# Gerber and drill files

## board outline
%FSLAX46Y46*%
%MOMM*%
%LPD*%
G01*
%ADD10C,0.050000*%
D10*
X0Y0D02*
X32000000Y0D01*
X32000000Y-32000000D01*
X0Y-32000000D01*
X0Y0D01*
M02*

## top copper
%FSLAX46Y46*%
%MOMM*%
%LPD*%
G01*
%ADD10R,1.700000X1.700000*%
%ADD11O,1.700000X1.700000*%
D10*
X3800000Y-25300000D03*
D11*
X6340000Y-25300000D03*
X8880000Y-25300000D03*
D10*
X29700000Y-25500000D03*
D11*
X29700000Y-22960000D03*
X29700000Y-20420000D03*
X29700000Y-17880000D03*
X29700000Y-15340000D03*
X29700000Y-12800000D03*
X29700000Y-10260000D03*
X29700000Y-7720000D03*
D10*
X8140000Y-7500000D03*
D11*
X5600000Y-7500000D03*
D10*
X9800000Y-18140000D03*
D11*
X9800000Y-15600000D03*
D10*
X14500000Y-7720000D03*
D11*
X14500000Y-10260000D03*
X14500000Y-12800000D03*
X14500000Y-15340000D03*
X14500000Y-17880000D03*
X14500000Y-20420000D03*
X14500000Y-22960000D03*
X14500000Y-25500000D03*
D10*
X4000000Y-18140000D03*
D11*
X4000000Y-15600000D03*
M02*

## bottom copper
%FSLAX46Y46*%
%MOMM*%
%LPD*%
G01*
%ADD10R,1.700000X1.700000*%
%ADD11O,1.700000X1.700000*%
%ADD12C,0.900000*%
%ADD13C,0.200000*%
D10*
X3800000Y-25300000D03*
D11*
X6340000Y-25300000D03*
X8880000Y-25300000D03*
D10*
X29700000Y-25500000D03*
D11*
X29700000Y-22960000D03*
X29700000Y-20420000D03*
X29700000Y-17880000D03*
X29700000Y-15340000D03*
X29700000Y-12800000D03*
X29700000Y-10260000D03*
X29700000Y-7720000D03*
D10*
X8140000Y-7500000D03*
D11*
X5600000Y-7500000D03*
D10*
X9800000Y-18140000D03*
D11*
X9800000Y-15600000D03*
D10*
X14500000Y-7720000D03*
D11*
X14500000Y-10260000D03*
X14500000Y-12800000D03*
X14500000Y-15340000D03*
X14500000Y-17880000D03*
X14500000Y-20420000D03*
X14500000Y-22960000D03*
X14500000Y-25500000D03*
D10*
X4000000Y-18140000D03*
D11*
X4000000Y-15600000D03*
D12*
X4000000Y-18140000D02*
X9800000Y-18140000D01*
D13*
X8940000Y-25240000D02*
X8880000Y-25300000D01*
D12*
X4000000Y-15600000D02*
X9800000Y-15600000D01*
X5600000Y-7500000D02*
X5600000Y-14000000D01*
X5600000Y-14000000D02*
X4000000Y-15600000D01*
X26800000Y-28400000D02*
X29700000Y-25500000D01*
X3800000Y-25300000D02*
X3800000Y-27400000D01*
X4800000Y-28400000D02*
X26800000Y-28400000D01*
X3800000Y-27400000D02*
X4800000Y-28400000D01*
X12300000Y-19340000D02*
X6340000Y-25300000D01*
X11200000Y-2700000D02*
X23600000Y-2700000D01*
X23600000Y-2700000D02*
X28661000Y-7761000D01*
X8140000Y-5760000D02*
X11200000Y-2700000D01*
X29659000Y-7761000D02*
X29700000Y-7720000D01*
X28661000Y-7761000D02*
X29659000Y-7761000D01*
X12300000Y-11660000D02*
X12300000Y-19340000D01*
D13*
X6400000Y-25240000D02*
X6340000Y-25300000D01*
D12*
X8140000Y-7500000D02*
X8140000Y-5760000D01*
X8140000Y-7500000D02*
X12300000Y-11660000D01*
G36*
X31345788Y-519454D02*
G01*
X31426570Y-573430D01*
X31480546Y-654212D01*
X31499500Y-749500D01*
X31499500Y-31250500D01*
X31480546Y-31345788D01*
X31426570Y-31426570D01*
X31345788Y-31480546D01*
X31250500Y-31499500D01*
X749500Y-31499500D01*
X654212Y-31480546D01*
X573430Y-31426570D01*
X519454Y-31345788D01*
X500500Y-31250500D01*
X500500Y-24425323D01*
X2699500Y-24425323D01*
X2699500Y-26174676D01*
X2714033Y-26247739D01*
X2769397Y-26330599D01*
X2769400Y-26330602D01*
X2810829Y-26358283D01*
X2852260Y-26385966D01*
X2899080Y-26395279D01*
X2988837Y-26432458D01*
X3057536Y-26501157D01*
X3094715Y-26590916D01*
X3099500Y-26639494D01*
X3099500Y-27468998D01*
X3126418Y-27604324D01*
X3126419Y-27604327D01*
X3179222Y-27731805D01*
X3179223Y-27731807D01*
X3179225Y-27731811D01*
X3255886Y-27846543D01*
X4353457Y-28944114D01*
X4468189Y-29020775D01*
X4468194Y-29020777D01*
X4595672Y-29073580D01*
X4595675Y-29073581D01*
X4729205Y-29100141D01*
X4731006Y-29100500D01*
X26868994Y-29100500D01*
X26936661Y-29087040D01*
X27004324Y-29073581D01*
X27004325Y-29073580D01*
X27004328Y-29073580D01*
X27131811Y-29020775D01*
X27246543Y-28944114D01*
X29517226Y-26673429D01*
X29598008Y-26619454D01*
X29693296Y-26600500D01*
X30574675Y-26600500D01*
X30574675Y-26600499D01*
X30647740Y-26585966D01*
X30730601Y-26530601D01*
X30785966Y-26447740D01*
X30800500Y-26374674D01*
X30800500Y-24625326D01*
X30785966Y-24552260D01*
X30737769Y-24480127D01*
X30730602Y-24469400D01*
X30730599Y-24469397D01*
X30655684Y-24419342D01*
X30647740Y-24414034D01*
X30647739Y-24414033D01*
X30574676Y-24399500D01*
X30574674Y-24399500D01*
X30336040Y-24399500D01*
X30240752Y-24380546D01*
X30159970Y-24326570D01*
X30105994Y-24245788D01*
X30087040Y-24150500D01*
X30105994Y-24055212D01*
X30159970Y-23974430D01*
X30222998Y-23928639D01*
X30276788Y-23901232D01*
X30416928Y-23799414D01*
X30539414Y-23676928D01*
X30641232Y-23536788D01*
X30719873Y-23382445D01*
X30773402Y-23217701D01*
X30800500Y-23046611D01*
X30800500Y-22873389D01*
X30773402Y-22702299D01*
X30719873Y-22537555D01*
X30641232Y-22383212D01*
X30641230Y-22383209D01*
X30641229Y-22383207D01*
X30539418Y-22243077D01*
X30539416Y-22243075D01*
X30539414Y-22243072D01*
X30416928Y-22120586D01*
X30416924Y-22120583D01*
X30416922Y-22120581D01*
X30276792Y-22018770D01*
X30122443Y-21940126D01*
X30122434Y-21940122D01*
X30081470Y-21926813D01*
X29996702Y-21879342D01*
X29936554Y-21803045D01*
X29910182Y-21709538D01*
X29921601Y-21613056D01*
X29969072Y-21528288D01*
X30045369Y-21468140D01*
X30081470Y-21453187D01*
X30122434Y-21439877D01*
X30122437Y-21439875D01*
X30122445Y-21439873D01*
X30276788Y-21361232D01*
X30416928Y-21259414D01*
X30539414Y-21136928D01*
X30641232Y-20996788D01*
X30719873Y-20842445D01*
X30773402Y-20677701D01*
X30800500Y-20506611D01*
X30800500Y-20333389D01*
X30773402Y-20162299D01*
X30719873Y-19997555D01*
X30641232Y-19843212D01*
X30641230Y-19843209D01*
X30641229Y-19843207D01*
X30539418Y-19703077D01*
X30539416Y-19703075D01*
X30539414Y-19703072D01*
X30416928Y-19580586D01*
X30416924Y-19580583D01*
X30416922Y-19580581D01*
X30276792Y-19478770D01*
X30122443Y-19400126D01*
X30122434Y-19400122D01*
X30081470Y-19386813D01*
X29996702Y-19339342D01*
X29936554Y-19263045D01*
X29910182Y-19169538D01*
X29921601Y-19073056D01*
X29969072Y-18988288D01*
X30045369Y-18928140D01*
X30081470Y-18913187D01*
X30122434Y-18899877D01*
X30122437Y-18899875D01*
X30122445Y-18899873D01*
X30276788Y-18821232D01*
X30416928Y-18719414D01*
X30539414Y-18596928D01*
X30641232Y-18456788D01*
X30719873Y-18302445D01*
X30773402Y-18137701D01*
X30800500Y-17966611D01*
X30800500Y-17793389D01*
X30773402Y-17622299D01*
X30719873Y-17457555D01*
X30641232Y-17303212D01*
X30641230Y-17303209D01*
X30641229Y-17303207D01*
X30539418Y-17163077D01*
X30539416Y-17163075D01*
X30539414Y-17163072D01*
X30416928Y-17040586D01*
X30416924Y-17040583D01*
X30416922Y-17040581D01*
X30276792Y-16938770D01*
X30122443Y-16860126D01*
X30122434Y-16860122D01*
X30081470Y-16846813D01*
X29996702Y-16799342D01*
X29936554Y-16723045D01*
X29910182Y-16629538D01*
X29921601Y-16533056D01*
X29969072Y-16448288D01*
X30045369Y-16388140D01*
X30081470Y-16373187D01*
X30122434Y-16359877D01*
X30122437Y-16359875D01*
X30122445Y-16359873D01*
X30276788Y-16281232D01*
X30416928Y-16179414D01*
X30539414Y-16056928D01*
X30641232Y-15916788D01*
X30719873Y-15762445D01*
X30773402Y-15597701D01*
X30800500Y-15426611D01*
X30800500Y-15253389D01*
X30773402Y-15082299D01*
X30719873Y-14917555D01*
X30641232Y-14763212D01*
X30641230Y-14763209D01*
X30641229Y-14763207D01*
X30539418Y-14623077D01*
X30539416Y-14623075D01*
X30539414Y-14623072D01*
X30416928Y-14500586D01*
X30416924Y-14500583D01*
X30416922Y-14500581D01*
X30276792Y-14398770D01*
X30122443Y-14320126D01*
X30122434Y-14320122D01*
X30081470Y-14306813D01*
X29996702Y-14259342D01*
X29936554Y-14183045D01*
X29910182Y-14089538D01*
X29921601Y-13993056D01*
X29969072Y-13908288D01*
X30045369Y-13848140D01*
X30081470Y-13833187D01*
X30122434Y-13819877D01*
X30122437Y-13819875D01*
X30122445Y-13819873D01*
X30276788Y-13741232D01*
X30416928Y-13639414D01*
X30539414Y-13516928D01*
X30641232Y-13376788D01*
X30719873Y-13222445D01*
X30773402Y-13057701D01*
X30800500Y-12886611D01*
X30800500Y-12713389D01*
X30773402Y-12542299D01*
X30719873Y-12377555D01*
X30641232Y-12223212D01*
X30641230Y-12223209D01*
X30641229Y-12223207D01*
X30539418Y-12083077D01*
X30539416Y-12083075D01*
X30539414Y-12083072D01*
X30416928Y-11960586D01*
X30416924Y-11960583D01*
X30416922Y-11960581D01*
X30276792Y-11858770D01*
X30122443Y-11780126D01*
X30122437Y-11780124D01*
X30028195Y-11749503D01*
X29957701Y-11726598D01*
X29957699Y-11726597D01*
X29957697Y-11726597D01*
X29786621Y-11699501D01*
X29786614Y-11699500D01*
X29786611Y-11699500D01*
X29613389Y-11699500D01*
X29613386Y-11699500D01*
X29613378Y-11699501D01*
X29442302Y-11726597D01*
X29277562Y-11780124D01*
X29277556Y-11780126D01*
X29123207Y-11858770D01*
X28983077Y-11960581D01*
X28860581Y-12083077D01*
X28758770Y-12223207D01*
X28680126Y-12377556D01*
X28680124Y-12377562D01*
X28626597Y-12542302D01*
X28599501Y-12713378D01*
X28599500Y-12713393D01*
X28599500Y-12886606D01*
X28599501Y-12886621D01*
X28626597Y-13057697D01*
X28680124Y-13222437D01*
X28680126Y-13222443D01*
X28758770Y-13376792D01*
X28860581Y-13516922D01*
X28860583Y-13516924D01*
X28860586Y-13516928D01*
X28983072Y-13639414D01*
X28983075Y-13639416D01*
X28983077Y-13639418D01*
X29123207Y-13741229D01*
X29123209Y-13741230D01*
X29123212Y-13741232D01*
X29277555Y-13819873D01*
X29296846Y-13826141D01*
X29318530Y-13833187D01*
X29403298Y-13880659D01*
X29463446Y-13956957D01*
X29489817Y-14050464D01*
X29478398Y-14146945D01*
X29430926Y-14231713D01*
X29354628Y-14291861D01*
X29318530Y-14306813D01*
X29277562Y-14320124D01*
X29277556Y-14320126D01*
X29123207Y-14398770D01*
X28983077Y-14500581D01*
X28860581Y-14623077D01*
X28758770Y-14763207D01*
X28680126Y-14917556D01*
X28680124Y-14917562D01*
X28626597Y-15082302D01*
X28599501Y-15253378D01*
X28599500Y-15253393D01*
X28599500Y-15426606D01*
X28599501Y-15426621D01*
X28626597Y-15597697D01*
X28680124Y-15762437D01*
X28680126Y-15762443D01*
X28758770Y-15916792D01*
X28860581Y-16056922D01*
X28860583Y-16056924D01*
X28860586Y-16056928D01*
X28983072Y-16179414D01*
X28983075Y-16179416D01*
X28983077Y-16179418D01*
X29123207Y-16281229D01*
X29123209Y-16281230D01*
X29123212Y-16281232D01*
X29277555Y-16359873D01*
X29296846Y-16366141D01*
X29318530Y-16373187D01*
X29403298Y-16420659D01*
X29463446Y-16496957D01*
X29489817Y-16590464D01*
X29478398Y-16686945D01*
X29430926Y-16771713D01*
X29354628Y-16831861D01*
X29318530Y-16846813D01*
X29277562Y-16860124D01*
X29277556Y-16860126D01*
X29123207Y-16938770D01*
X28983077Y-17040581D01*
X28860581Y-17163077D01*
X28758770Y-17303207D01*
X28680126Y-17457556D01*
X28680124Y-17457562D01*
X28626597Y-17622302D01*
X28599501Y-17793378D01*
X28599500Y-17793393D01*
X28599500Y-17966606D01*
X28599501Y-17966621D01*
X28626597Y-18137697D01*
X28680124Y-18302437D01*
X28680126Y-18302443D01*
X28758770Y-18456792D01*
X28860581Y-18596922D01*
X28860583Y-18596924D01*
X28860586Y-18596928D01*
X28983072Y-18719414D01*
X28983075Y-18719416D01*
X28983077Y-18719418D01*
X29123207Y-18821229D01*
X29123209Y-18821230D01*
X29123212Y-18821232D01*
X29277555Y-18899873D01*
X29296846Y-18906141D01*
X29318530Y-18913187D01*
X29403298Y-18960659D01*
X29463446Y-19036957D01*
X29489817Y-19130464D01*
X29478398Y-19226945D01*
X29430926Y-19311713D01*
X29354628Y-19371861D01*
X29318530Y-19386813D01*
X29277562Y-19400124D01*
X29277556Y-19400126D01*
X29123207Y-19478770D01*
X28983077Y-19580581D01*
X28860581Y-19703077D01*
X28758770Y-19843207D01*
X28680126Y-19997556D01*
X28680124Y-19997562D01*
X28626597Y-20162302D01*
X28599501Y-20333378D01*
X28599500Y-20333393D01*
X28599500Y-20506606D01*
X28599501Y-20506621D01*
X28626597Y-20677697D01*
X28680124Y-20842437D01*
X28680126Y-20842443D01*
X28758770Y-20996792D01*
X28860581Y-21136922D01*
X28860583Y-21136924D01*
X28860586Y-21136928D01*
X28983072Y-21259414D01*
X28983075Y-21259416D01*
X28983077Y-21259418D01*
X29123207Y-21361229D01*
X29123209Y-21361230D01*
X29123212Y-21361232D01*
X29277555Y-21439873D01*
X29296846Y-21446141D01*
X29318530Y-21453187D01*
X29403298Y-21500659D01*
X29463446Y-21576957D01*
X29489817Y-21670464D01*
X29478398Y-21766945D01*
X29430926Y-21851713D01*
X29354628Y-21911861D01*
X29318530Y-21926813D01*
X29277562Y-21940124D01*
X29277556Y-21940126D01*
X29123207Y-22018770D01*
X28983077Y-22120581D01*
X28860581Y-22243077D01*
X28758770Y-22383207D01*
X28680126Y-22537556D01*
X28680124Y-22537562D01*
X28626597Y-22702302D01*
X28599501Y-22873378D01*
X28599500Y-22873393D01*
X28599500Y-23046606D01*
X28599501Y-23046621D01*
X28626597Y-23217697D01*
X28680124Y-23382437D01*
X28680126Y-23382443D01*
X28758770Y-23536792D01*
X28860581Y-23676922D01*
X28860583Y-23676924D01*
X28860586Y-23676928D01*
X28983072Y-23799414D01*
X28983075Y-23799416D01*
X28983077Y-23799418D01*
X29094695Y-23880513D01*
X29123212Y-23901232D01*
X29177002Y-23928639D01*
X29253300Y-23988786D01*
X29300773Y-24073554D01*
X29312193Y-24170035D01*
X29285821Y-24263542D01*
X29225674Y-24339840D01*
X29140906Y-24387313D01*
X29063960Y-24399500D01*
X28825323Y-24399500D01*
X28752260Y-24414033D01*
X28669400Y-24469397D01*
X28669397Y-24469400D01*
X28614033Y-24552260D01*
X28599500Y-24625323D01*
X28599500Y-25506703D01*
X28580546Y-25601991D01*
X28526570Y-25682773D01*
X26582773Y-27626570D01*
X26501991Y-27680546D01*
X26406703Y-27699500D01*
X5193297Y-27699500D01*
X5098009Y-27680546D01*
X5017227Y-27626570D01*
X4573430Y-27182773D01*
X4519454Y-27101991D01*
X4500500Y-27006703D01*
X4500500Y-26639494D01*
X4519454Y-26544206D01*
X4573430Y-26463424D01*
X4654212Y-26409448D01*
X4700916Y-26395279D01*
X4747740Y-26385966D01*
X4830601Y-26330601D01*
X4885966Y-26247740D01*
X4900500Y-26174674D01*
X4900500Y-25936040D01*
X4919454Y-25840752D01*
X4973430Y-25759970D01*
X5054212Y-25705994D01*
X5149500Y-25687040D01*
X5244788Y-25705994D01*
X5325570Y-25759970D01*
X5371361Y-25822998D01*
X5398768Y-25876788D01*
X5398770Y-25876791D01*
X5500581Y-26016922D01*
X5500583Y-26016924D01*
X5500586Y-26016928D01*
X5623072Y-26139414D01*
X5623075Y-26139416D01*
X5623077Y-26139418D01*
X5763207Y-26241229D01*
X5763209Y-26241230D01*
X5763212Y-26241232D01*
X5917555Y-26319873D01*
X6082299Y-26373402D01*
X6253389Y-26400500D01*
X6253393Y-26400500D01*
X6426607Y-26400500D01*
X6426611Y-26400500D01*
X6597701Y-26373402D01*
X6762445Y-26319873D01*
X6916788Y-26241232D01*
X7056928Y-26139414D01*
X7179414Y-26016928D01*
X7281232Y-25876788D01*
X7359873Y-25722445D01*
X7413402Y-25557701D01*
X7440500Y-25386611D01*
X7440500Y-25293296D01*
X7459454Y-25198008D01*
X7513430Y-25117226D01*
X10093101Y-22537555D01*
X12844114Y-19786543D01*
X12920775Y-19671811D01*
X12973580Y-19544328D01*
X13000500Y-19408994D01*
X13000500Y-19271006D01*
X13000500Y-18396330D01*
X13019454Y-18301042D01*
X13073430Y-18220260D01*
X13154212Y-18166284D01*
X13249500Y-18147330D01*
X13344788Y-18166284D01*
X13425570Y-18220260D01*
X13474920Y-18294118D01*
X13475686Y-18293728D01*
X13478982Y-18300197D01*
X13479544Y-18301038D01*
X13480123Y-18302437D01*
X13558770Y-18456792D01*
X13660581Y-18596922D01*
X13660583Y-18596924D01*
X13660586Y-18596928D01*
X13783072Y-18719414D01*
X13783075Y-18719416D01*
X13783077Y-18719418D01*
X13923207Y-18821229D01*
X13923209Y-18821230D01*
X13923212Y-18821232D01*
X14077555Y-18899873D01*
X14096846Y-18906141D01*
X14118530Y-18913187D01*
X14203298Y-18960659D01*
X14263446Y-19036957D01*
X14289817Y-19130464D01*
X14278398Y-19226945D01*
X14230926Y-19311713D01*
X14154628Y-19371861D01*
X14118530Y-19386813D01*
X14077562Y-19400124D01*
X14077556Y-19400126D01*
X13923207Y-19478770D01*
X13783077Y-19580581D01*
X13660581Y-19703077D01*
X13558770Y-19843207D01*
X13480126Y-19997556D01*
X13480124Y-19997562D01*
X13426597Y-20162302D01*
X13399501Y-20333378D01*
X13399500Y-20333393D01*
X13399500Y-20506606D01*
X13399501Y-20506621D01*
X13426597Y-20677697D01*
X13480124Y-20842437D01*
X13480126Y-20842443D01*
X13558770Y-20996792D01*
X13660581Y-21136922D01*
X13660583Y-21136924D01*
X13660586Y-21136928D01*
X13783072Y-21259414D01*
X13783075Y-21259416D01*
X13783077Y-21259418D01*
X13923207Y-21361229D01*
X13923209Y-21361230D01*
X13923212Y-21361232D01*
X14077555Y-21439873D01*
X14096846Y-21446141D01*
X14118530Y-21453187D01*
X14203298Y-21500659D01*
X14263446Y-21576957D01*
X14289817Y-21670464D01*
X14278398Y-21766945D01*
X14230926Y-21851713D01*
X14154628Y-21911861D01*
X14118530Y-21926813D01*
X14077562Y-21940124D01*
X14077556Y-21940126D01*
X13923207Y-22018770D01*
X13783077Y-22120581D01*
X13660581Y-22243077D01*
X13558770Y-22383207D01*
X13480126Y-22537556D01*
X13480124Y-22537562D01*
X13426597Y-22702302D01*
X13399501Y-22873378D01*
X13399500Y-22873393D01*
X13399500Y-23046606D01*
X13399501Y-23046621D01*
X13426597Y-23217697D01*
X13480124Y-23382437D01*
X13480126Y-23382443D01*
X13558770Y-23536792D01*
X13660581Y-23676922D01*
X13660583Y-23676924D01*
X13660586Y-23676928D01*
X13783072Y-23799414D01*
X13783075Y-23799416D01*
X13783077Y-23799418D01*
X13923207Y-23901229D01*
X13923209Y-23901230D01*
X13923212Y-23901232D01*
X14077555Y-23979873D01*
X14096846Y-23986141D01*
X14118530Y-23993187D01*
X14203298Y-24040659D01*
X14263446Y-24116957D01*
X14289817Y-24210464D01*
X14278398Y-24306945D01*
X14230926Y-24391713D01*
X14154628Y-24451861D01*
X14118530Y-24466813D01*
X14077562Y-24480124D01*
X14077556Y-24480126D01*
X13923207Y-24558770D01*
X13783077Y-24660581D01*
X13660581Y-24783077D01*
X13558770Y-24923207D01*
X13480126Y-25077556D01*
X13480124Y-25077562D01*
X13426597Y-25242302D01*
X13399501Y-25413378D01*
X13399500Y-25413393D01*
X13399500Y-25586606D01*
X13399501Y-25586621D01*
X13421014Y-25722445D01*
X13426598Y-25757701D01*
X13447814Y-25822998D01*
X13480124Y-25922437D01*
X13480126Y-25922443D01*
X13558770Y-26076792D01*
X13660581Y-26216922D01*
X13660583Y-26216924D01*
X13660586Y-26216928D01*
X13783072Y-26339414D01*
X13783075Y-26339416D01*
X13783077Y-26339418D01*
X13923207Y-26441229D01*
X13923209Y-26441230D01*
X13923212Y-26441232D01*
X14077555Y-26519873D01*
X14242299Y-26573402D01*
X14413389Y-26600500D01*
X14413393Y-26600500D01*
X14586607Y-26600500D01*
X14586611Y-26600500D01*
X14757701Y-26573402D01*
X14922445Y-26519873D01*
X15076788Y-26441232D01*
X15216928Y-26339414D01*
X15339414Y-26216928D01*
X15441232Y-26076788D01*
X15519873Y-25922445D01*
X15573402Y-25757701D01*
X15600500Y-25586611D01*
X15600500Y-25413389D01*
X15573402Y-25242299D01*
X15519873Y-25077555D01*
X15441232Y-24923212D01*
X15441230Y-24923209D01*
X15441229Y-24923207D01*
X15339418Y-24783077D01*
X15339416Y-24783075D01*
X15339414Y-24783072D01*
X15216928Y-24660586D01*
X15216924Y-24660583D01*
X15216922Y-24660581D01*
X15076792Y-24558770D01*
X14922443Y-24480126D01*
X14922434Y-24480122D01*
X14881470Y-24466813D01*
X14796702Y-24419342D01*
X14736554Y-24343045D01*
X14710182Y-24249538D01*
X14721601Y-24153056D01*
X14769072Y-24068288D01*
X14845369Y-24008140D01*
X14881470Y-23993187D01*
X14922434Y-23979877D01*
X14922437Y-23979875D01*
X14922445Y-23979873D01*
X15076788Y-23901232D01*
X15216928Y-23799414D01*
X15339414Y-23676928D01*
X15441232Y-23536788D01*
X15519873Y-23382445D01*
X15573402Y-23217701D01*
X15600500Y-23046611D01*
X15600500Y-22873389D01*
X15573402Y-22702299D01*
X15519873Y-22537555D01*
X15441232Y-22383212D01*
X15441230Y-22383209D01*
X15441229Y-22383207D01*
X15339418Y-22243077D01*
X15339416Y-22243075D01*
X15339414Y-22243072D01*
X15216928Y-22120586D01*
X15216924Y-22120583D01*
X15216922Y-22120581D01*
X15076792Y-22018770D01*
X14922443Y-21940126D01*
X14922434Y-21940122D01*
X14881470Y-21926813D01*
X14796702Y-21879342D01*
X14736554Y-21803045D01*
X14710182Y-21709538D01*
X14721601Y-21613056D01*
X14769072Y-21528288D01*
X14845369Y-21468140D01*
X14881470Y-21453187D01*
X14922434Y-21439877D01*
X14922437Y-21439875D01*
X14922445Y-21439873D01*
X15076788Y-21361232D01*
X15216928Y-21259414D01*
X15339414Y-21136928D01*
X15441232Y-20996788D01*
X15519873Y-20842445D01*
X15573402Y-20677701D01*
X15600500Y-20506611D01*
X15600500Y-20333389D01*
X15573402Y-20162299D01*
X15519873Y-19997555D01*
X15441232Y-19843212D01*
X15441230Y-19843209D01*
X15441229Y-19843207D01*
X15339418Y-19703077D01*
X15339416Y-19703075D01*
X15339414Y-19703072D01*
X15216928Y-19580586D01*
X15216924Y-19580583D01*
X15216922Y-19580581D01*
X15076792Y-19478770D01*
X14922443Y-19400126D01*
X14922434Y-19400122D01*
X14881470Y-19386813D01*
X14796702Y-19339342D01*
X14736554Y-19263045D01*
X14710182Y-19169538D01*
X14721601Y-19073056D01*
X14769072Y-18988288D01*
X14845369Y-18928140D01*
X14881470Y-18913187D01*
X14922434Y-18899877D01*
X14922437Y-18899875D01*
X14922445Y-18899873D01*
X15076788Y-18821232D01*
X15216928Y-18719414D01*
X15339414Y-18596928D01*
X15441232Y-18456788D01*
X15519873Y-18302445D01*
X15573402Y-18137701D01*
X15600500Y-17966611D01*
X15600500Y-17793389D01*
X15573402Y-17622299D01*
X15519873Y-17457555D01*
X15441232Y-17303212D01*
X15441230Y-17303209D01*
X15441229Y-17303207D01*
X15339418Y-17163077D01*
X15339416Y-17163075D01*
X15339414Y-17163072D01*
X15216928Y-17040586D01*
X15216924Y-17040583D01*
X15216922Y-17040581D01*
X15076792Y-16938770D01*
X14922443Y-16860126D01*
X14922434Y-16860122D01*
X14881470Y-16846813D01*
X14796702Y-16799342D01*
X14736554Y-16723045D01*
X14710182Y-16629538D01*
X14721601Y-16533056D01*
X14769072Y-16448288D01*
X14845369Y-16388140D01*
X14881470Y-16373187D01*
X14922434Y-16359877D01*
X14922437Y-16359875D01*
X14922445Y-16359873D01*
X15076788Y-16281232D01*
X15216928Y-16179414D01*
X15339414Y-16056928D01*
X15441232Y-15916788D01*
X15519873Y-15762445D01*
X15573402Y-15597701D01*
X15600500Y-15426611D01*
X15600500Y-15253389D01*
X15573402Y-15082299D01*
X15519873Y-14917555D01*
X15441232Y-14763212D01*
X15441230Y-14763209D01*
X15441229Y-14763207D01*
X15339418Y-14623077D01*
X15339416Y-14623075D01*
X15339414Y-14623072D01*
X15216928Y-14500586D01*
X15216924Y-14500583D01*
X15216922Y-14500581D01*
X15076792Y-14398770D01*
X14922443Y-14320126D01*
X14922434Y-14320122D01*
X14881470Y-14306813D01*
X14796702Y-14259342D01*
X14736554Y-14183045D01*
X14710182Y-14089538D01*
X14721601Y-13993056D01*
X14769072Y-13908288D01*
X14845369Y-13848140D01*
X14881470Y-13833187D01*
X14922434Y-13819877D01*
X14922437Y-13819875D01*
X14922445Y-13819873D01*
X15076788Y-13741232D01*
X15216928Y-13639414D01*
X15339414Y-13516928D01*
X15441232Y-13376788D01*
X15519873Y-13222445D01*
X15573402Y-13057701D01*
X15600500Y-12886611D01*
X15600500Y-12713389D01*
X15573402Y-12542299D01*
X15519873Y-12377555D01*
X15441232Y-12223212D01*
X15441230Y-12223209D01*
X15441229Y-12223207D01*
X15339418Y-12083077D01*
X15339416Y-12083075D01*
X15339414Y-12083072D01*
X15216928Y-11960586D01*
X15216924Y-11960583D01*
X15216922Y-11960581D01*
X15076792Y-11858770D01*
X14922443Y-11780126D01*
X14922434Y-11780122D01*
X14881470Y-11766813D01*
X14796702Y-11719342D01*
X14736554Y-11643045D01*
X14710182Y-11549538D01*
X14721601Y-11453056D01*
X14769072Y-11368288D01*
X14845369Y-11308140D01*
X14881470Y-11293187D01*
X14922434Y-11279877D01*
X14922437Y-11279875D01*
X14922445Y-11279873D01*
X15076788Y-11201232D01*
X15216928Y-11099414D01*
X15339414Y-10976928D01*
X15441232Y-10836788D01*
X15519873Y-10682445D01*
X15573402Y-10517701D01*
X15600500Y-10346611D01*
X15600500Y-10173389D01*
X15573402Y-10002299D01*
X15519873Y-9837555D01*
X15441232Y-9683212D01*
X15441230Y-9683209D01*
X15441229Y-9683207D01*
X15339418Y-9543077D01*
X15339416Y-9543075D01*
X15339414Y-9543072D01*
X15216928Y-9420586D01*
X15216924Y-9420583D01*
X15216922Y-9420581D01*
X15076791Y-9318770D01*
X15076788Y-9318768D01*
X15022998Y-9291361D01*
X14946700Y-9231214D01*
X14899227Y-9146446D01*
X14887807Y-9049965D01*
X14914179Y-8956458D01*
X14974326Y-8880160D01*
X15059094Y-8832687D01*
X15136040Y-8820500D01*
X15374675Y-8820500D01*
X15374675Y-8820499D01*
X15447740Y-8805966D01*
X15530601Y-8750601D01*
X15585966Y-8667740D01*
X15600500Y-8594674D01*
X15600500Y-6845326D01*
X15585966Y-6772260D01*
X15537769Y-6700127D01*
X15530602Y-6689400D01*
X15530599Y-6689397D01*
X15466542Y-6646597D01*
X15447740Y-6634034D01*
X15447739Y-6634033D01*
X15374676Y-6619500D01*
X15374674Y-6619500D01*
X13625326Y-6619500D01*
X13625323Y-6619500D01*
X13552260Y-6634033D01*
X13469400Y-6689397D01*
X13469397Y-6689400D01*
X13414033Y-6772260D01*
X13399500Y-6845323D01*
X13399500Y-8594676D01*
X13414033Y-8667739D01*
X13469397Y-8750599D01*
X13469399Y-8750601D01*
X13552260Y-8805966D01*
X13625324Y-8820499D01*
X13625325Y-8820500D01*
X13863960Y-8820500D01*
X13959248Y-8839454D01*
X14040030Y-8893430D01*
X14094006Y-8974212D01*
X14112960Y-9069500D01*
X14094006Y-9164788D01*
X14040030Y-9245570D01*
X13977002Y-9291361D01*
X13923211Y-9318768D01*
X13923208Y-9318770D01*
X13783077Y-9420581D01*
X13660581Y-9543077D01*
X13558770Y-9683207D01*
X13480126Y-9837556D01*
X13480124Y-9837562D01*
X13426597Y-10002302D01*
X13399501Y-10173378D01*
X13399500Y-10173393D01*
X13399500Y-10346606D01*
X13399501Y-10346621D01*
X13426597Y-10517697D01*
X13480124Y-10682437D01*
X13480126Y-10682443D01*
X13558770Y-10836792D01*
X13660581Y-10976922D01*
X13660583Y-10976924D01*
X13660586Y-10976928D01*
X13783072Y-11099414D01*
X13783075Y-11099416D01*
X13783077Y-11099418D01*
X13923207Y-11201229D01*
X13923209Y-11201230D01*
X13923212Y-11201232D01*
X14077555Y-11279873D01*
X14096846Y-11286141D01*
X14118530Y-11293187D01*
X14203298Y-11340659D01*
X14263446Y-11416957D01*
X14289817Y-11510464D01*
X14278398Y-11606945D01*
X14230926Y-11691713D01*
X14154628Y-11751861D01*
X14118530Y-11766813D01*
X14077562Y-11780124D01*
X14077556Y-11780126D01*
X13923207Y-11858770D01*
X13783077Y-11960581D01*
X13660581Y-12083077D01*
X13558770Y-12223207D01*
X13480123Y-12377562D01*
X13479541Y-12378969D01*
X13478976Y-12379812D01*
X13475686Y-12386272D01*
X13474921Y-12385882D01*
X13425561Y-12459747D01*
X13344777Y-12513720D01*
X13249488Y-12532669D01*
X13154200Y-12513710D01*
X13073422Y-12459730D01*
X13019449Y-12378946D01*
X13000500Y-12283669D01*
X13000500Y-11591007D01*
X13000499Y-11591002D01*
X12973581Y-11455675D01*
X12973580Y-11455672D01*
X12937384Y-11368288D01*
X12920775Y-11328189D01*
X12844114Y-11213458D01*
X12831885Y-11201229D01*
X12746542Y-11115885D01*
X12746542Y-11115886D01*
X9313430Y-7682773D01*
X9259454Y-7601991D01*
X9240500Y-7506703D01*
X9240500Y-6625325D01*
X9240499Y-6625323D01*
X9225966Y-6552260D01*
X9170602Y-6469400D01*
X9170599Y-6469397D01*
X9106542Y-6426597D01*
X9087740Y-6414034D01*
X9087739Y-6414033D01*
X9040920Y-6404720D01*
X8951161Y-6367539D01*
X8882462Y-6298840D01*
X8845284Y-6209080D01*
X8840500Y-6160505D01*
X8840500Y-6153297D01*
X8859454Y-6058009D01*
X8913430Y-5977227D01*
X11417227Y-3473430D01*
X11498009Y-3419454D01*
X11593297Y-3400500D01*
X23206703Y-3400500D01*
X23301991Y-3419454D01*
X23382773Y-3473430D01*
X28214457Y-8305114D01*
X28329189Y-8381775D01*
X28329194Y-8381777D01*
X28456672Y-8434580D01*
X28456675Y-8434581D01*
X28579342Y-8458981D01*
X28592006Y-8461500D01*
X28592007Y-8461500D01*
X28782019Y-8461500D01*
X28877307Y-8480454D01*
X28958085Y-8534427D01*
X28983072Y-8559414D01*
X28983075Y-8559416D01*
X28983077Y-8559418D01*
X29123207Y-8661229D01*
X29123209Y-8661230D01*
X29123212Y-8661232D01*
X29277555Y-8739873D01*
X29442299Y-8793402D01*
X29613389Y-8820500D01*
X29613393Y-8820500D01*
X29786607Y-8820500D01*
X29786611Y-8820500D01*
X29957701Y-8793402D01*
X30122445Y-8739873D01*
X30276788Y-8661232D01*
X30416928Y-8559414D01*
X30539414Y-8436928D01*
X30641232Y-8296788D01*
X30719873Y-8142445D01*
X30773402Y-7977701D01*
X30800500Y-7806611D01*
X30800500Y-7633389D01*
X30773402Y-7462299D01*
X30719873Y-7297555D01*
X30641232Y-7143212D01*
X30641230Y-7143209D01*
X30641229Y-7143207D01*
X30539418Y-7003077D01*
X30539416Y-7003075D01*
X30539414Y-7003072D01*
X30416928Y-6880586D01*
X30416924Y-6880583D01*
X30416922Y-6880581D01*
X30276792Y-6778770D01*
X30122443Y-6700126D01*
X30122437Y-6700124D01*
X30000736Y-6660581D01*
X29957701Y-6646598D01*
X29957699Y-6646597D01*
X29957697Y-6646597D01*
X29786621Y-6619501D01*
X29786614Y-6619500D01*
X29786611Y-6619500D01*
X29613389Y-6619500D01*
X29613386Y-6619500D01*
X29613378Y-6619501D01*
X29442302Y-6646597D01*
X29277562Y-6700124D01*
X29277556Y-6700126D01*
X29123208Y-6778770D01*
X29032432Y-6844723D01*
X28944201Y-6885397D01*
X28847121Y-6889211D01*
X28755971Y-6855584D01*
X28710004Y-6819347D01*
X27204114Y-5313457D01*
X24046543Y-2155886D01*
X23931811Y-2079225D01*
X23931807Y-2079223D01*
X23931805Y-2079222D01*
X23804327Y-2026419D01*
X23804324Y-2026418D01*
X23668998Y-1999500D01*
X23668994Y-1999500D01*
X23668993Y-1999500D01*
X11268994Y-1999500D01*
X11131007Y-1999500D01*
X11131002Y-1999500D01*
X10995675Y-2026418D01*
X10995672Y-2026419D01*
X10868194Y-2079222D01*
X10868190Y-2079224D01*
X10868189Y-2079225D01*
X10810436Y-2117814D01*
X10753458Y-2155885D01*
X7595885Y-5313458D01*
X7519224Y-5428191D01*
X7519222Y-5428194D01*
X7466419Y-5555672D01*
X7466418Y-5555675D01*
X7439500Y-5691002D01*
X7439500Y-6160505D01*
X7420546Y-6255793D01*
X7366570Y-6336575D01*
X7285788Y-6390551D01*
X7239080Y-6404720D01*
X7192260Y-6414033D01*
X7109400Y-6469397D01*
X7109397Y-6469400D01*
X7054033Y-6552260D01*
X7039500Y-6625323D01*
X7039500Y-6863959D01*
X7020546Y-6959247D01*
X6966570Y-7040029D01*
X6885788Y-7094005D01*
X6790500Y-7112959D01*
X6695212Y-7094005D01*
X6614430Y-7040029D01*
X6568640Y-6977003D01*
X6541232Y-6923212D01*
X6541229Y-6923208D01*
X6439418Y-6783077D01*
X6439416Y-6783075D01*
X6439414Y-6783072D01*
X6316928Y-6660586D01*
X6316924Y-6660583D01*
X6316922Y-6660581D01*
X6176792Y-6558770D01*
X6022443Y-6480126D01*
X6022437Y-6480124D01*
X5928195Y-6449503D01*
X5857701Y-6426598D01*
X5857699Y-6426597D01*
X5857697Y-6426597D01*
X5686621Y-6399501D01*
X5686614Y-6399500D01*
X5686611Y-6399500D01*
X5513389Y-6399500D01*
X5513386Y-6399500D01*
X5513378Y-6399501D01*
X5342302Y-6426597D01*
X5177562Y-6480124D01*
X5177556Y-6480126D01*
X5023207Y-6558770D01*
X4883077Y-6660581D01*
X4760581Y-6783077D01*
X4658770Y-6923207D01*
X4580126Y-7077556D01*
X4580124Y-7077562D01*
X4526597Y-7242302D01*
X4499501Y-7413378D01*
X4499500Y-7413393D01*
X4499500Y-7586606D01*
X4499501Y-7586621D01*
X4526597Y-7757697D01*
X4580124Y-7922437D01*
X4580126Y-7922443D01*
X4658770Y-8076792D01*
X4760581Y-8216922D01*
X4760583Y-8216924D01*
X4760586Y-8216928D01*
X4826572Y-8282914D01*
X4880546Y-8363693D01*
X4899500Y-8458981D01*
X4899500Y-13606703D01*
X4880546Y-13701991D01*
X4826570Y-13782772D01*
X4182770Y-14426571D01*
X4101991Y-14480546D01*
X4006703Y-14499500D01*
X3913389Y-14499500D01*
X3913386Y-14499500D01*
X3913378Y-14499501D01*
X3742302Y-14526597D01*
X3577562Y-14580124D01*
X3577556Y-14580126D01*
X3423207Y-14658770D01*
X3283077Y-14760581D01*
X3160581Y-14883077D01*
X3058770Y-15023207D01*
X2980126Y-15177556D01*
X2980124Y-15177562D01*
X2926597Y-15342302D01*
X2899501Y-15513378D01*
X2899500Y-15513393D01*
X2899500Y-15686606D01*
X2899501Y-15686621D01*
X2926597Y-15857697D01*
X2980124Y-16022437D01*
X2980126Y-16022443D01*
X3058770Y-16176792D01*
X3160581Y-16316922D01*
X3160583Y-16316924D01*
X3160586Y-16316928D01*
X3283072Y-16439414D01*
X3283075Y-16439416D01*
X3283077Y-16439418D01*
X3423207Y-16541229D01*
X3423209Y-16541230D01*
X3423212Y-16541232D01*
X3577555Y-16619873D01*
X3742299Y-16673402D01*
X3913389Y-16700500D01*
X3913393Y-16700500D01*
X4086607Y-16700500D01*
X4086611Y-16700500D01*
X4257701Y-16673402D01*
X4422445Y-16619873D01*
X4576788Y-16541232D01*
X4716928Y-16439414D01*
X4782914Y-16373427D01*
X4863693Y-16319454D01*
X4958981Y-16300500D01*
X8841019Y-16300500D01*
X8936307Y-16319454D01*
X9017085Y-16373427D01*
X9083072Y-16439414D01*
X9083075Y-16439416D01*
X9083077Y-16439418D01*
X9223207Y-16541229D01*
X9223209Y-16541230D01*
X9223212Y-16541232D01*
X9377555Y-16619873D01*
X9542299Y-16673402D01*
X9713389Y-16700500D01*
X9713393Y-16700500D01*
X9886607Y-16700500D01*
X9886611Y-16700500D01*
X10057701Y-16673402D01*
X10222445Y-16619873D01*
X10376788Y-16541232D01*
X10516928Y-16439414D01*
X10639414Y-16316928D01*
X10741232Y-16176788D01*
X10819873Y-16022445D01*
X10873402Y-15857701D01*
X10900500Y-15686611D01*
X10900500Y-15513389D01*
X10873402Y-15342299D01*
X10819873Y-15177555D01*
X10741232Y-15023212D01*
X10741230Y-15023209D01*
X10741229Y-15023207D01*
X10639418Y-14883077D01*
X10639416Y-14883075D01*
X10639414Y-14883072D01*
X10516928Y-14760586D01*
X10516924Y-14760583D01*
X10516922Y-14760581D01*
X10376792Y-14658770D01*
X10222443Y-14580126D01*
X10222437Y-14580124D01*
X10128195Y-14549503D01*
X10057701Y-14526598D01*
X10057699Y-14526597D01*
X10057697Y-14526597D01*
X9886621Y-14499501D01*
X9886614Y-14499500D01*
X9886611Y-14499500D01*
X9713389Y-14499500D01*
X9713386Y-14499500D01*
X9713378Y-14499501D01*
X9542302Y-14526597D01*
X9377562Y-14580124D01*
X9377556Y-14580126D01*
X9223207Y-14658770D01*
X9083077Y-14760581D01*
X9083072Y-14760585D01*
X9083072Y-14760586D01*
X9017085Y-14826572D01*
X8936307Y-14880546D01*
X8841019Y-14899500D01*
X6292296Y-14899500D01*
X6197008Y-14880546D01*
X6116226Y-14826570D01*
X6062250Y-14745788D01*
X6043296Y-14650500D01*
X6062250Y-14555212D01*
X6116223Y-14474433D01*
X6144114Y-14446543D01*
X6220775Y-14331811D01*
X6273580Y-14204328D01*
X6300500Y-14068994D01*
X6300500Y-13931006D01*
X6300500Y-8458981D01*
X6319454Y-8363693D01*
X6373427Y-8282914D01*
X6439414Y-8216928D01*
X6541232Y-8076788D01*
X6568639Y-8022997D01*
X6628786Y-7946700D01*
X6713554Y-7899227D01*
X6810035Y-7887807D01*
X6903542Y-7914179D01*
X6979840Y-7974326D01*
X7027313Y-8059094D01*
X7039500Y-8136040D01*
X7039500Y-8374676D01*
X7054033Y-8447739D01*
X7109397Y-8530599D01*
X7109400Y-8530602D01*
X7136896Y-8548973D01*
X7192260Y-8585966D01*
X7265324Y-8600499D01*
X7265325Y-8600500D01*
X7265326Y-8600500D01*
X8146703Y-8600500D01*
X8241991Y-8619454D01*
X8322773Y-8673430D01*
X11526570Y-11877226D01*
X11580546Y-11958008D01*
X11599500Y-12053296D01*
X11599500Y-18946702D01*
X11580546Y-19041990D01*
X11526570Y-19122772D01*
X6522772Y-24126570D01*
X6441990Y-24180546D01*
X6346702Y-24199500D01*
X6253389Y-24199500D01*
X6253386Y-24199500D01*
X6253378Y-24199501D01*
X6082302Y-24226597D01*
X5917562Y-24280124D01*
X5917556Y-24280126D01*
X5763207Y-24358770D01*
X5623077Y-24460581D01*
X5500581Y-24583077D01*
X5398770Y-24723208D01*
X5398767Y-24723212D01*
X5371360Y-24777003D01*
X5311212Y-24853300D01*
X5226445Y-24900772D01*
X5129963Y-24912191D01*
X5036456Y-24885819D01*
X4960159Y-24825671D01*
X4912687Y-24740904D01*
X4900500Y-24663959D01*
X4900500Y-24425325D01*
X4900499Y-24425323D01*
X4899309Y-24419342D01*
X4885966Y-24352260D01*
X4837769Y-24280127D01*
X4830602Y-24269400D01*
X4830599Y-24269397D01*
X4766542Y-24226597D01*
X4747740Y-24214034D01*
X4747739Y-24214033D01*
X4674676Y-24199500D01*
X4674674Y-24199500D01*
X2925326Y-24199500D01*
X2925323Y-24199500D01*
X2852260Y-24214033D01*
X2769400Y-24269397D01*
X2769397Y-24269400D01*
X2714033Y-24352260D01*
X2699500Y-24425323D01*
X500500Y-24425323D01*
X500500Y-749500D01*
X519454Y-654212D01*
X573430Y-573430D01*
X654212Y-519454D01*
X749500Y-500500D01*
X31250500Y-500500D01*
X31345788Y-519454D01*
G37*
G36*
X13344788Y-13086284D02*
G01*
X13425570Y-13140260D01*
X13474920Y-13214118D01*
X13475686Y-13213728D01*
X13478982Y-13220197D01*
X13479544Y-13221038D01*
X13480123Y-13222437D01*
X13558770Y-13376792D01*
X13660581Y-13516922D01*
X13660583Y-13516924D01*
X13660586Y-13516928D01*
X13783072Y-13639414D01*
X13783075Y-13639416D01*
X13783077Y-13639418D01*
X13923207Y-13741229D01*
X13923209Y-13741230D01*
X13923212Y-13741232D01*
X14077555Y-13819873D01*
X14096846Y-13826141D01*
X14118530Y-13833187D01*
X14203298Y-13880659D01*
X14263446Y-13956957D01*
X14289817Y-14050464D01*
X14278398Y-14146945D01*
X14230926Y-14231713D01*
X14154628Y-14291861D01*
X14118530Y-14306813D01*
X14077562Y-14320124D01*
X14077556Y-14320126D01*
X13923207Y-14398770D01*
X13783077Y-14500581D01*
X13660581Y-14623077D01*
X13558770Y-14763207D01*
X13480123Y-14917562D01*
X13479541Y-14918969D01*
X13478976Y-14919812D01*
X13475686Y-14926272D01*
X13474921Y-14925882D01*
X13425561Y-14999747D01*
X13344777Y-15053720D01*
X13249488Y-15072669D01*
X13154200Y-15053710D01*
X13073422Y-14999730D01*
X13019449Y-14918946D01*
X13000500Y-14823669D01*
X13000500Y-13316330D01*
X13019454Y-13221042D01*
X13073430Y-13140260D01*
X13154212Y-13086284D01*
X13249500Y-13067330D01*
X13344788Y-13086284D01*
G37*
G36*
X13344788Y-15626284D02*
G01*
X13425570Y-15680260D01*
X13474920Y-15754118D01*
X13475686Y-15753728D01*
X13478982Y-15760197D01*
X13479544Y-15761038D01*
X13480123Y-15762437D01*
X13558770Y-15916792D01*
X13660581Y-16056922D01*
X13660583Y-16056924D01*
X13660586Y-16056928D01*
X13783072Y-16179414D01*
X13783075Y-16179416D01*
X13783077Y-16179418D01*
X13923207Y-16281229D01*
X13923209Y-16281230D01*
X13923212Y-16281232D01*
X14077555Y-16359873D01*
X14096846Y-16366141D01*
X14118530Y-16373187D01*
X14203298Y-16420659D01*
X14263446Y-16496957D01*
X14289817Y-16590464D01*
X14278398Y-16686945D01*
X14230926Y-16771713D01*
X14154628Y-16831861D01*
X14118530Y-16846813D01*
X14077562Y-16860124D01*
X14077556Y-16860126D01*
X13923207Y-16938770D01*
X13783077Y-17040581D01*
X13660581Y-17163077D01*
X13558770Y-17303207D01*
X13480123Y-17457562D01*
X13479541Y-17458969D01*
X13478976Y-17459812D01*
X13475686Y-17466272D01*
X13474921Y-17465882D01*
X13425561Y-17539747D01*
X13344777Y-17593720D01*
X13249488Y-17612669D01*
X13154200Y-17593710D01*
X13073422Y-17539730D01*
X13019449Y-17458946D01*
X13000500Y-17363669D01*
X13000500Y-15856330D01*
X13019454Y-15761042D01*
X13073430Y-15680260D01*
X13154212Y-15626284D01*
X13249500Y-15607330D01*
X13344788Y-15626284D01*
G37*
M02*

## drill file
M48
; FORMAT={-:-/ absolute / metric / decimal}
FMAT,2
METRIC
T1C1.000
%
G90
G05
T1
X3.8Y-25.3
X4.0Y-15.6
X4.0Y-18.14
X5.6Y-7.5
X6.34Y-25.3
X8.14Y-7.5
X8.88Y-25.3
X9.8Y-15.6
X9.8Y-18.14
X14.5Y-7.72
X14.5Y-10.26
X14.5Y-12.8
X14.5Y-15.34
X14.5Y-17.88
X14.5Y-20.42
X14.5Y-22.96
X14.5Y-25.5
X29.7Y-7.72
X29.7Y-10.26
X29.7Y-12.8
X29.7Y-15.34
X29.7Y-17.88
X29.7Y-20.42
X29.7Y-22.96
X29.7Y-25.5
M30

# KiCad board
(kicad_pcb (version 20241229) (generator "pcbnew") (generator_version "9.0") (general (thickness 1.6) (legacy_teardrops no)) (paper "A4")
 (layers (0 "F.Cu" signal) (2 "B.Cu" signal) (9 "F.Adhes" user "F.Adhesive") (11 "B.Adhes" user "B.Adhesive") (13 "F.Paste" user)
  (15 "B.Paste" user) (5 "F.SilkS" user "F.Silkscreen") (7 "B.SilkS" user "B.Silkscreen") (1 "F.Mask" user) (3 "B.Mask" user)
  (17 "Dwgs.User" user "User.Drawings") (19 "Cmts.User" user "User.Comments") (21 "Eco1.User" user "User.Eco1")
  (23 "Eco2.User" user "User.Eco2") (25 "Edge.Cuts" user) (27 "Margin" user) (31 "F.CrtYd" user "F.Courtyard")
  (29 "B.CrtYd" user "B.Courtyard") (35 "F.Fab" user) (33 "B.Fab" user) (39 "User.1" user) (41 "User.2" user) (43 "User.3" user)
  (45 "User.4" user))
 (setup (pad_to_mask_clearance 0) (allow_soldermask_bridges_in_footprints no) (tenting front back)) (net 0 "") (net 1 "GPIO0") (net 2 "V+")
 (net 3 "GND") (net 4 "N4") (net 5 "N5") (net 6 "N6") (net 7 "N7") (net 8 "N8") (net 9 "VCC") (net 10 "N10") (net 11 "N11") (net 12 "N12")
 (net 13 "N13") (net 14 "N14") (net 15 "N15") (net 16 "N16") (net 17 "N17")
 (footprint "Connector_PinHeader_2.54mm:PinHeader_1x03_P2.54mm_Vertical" (layer "F.Cu") (at 3.8 25.3 90)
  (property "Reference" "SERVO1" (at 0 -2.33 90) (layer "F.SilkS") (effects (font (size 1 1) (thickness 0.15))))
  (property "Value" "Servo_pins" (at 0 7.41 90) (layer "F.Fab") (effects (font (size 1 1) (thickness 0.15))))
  (pad "1" thru_hole rect (at 0 0 90) (size 1.7 1.7) (drill 1) (layers "*.Cu" "*.Mask") (remove_unused_layers no) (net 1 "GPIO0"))
  (pad "2" thru_hole oval (at 0 2.54 90) (size 1.7 1.7) (drill 1) (layers "*.Cu" "*.Mask") (remove_unused_layers no) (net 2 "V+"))
  (pad "3" thru_hole oval (at 0 5.08 90) (size 1.7 1.7) (drill 1) (layers "*.Cu" "*.Mask") (remove_unused_layers no) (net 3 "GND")))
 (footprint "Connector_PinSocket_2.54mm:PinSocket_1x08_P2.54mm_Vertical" (layer "F.Cu") (at 29.7 25.5 180)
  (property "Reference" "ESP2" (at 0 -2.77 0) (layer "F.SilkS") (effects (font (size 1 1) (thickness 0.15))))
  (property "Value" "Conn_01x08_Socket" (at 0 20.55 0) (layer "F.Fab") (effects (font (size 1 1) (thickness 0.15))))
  (pad "1" thru_hole rect (at 0 0 180) (size 1.7 1.7) (drill 1) (layers "*.Cu" "*.Mask") (remove_unused_layers no) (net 1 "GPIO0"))
  (pad "2" thru_hole oval (at 0 2.54 180) (size 1.7 1.7) (drill 1) (layers "*.Cu" "*.Mask") (remove_unused_layers no) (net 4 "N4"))
  (pad "3" thru_hole oval (at 0 5.08 180) (size 1.7 1.7) (drill 1) (layers "*.Cu" "*.Mask") (remove_unused_layers no) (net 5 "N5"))
  (pad "4" thru_hole oval (at 0 7.62 180) (size 1.7 1.7) (drill 1) (layers "*.Cu" "*.Mask") (remove_unused_layers no) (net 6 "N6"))
  (pad "5" thru_hole oval (at 0 10.16 180) (size 1.7 1.7) (drill 1) (layers "*.Cu" "*.Mask") (remove_unused_layers no) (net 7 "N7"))
  (pad "6" thru_hole oval (at 0 12.7 180) (size 1.7 1.7) (drill 1) (layers "*.Cu" "*.Mask") (remove_unused_layers no) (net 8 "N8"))
  (pad "7" thru_hole oval (at 0 15.24 180) (size 1.7 1.7) (drill 1) (layers "*.Cu" "*.Mask") (remove_unused_layers no) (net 3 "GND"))
  (pad "8" thru_hole oval (at 0 17.78 180) (size 1.7 1.7) (drill 1) (layers "*.Cu" "*.Mask") (remove_unused_layers no) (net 2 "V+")))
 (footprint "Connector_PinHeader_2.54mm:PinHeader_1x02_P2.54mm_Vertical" (layer "F.Cu") (at 8.14 7.5 -90)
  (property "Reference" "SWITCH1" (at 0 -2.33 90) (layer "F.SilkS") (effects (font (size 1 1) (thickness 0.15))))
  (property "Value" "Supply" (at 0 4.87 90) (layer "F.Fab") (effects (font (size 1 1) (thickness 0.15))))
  (pad "1" thru_hole rect (at 0 0 270) (size 1.7 1.7) (drill 1) (layers "*.Cu" "*.Mask") (remove_unused_layers no) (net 2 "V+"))
  (pad "2" thru_hole oval (at 0 2.54 270) (size 1.7 1.7) (drill 1) (layers "*.Cu" "*.Mask") (remove_unused_layers no) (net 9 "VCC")))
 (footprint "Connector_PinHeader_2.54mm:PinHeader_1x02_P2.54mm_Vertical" (layer "F.Cu") (at 9.8 18.14 180)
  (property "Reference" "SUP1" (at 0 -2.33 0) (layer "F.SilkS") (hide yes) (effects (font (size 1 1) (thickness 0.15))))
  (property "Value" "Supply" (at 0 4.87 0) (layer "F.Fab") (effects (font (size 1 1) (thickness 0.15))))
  (pad "1" thru_hole rect (at 0 0 180) (size 1.7 1.7) (drill 1) (layers "*.Cu" "*.Mask") (remove_unused_layers no) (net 3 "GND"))
  (pad "2" thru_hole oval (at 0 2.54 180) (size 1.7 1.7) (drill 1) (layers "*.Cu" "*.Mask") (remove_unused_layers no) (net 9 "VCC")))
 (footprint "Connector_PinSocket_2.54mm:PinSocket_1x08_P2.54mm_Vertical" (layer "F.Cu") (at 14.5 7.72)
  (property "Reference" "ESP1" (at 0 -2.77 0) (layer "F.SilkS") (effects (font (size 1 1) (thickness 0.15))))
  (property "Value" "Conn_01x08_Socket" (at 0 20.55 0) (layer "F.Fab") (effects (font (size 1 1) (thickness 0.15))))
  (pad "1" thru_hole rect (at 0 0) (size 1.7 1.7) (drill 1) (layers "*.Cu" "*.Mask") (remove_unused_layers no) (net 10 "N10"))
  (pad "2" thru_hole oval (at 0 2.54) (size 1.7 1.7) (drill 1) (layers "*.Cu" "*.Mask") (remove_unused_layers no) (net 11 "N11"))
  (pad "3" thru_hole oval (at 0 5.08) (size 1.7 1.7) (drill 1) (layers "*.Cu" "*.Mask") (remove_unused_layers no) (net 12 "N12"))
  (pad "4" thru_hole oval (at 0 7.62) (size 1.7 1.7) (drill 1) (layers "*.Cu" "*.Mask") (remove_unused_layers no) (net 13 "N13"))
  (pad "5" thru_hole oval (at 0 10.16) (size 1.7 1.7) (drill 1) (layers "*.Cu" "*.Mask") (remove_unused_layers no) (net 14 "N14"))
  (pad "6" thru_hole oval (at 0 12.7) (size 1.7 1.7) (drill 1) (layers "*.Cu" "*.Mask") (remove_unused_layers no) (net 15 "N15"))
  (pad "7" thru_hole oval (at 0 15.24) (size 1.7 1.7) (drill 1) (layers "*.Cu" "*.Mask") (remove_unused_layers no) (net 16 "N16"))
  (pad "8" thru_hole oval (at 0 17.78) (size 1.7 1.7) (drill 1) (layers "*.Cu" "*.Mask") (remove_unused_layers no) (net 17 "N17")))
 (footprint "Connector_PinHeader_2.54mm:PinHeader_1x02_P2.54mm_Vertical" (layer "F.Cu") (at 4 18.14 180)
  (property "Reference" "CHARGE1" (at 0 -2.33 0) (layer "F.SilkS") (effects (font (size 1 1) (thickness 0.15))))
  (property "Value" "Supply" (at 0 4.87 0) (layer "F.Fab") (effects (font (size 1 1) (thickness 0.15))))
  (pad "1" thru_hole rect (at 0 0 180) (size 1.7 1.7) (drill 1) (layers "*.Cu" "*.Mask") (remove_unused_layers no) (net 3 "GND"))
  (pad "2" thru_hole oval (at 0 2.54 180) (size 1.7 1.7) (drill 1) (layers "*.Cu" "*.Mask") (remove_unused_layers no) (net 9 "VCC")))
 (gr_rect (start 0 0) (end 32 32) (stroke (width 0.05) (type solid)) (fill no) (layer "Edge.Cuts"))
 (segment (start 4 18.14) (end 9.8 18.14) (width 0.9) (layer "B.Cu") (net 3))
 (segment (start 8.94 25.24) (end 8.88 25.3) (width 0.2) (layer "B.Cu") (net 3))
 (segment (start 4 15.6) (end 9.8 15.6) (width 0.9) (layer "B.Cu") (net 9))
 (segment (start 5.6 7.5) (end 5.6 14) (width 0.9) (layer "B.Cu") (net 9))
 (segment (start 5.6 14) (end 4 15.6) (width 0.9) (layer "B.Cu") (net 9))
 (segment (start 26.8 28.4) (end 29.7 25.5) (width 0.9) (layer "B.Cu") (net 1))
 (segment (start 3.8 25.3) (end 3.8 27.4) (width 0.9) (layer "B.Cu") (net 1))
 (segment (start 4.8 28.4) (end 26.8 28.4) (width 0.9) (layer "B.Cu") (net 1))
 (segment (start 3.8 27.4) (end 4.8 28.4) (width 0.9) (layer "B.Cu") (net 1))
 (segment (start 12.3 19.34) (end 6.34 25.3) (width 0.9) (layer "B.Cu") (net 2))
 (segment (start 11.2 2.7) (end 23.6 2.7) (width 0.9) (layer "B.Cu") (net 2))
 (segment (start 23.6 2.7) (end 28.661 7.761) (width 0.9) (layer "B.Cu") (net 2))
 (segment (start 8.14 5.76) (end 11.2 2.7) (width 0.9) (layer "B.Cu") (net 2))
 (segment (start 29.659 7.761) (end 29.7 7.72) (width 0.9) (layer "B.Cu") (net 2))
 (segment (start 28.661 7.761) (end 29.659 7.761) (width 0.9) (layer "B.Cu") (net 2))
 (segment (start 12.3 11.66) (end 12.3 19.34) (width 0.9) (layer "B.Cu") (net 2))
 (segment (start 6.4 25.24) (end 6.34 25.3) (width 0.2) (layer "B.Cu") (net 2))
 (segment (start 8.14 7.5) (end 8.14 5.76) (width 0.9) (layer "B.Cu") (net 2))
 (segment (start 8.14 7.5) (end 12.3 11.66) (width 0.9) (layer "B.Cu") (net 2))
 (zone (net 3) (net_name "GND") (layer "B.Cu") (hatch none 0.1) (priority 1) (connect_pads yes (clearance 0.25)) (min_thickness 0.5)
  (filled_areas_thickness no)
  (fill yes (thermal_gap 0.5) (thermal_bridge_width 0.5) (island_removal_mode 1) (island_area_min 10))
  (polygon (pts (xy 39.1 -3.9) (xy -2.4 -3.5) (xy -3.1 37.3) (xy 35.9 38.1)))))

